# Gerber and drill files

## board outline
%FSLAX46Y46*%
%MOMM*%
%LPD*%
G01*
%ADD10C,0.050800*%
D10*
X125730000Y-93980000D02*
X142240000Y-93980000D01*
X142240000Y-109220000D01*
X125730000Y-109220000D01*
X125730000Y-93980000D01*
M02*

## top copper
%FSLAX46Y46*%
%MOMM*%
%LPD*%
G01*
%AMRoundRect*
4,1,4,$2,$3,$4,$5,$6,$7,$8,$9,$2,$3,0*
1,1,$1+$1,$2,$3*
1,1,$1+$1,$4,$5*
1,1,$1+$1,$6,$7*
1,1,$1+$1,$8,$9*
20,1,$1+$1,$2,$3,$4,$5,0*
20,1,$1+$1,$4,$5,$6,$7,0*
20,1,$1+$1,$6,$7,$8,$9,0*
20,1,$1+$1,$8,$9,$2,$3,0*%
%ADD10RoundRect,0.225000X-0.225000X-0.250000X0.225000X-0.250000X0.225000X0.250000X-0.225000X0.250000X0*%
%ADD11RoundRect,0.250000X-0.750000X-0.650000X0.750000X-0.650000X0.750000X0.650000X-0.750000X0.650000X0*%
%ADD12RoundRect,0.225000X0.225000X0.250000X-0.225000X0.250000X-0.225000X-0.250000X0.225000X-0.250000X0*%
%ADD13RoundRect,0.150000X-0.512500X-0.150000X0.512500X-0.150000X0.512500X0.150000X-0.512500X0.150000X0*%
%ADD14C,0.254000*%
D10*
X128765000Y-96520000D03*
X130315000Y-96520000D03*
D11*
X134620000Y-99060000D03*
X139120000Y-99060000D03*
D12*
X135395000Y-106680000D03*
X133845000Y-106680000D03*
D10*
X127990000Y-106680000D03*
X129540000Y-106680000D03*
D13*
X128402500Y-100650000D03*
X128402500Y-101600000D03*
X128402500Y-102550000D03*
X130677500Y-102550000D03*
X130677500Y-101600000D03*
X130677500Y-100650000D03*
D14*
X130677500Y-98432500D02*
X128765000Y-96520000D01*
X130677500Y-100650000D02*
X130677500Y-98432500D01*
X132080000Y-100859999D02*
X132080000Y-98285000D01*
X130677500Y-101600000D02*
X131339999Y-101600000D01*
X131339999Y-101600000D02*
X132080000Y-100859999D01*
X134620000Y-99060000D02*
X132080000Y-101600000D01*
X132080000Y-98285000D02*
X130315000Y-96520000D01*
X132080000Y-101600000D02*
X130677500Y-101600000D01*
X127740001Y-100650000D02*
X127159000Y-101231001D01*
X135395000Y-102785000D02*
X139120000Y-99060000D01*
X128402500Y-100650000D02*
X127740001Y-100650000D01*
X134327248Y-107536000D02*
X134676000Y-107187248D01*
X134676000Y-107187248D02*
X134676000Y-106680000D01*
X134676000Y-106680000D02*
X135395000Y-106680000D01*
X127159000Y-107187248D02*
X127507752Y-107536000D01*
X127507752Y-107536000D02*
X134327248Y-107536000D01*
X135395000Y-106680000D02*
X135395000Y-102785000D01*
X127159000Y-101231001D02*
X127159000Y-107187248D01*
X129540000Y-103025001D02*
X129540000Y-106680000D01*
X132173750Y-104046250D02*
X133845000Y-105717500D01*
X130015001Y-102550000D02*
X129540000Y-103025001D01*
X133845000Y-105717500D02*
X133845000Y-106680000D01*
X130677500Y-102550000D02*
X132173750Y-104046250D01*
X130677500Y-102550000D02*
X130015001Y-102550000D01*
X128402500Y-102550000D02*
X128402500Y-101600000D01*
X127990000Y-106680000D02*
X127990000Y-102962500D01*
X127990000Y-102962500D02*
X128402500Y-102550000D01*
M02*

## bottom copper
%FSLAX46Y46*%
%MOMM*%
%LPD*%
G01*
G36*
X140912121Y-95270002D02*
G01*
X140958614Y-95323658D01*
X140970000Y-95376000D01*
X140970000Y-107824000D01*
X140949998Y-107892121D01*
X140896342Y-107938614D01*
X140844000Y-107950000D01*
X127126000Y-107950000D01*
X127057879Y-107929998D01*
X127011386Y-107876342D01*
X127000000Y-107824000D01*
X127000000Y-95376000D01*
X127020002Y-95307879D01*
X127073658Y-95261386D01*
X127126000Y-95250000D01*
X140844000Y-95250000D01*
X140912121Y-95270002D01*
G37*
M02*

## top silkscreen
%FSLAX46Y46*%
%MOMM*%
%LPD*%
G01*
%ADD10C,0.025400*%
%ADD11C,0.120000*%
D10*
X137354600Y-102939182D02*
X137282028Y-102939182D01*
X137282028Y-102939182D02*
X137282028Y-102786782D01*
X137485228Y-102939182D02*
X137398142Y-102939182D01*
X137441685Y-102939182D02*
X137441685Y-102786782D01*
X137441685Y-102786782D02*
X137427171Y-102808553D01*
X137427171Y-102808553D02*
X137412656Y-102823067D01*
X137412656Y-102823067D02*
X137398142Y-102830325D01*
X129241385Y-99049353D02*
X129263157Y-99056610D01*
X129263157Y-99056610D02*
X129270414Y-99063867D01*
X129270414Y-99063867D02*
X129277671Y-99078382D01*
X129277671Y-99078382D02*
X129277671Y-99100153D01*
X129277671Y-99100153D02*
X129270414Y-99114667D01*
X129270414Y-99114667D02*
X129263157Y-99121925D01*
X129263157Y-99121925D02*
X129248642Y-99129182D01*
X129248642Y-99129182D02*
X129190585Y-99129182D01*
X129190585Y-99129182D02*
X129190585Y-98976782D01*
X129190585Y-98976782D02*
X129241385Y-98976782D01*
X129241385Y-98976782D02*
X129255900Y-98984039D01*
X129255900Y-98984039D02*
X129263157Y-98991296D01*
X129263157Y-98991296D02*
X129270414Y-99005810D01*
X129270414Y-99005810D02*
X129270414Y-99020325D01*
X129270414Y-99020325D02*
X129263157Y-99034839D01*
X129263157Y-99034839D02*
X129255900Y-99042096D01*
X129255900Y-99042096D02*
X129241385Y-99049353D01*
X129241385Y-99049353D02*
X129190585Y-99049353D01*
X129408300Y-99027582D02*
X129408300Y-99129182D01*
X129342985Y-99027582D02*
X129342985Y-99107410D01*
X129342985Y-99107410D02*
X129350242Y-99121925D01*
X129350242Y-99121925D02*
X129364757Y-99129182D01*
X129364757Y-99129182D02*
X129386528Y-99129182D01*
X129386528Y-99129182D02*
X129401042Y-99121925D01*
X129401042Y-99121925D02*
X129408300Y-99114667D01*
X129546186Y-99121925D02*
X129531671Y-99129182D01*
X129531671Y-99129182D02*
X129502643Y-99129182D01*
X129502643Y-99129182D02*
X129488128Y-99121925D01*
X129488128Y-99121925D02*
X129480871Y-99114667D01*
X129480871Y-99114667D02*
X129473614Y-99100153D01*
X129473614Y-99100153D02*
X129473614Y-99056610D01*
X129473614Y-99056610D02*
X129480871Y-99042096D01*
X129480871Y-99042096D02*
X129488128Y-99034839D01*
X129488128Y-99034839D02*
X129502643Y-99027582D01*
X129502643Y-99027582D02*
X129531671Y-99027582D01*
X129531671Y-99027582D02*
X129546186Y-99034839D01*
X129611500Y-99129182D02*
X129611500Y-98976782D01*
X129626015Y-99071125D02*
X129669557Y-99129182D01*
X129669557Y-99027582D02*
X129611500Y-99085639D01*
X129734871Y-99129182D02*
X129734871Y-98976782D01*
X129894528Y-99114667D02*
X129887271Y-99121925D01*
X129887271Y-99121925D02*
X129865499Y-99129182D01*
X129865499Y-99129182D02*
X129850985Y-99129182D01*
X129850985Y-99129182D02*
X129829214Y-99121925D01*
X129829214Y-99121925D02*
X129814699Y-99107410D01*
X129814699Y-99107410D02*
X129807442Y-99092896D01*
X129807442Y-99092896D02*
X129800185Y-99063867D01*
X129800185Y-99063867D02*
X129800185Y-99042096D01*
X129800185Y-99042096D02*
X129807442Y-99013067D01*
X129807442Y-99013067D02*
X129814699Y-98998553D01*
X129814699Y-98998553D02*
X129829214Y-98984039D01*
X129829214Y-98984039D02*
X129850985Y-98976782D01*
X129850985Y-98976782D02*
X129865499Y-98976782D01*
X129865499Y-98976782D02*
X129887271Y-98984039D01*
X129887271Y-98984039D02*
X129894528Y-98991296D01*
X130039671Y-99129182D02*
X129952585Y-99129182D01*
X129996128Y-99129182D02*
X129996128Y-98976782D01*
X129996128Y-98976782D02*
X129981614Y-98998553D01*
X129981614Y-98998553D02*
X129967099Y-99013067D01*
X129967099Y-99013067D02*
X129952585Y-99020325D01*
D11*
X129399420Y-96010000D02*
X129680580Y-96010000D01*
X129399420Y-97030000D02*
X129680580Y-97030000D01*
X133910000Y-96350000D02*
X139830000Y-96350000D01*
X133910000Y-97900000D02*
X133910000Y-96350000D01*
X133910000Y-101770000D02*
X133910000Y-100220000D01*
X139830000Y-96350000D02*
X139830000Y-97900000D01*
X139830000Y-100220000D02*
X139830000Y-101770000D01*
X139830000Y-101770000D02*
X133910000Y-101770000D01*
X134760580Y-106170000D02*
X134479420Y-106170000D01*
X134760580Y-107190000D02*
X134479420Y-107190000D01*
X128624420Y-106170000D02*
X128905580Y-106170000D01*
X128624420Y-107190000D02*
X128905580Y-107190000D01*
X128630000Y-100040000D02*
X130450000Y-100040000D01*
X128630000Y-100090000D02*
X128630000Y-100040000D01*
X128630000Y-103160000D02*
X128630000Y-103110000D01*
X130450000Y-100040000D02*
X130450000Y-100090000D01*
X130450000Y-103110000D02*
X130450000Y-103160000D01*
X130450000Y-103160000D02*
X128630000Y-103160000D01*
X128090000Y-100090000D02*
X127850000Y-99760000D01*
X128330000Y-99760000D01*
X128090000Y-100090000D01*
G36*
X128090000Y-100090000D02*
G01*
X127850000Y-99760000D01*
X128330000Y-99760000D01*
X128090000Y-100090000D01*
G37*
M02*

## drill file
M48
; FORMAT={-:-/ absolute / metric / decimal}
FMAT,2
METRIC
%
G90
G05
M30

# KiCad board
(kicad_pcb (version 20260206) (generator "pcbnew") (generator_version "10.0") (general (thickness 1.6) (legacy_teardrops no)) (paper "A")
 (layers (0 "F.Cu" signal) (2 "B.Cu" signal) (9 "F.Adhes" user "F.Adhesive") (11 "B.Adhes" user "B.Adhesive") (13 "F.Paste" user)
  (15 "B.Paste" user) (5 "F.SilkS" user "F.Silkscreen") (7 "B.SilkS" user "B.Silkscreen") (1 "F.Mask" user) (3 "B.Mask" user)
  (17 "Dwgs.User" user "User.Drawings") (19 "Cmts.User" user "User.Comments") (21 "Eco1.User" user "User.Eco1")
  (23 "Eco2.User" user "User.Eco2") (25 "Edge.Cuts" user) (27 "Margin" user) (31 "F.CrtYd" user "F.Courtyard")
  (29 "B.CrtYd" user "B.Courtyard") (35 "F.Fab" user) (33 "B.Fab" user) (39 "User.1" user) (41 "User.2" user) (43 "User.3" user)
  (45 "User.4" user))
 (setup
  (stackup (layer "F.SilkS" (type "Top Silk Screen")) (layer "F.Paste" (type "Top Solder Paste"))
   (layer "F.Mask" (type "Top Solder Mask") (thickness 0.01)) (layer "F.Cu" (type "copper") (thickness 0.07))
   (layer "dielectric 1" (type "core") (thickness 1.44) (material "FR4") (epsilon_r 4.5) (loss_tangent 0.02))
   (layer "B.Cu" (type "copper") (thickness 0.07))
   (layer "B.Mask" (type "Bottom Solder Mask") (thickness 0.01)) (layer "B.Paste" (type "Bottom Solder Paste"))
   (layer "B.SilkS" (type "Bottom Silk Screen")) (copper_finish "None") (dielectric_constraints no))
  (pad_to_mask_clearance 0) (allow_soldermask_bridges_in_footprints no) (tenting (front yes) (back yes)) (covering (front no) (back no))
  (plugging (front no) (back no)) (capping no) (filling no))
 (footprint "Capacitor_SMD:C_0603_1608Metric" (layer "F.Cu") (at 129.54 96.52)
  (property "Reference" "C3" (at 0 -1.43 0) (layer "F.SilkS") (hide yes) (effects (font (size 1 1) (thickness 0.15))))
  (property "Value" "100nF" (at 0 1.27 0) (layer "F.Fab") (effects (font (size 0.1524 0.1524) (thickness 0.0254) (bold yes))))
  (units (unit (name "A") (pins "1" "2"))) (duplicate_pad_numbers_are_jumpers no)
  (fp_line (start -0.14058 -0.51) (end 0.14058 -0.51) (stroke (width 0.12) (type solid)) (layer "F.SilkS"))
  (fp_line (start -0.14058 0.51) (end 0.14058 0.51) (stroke (width 0.12) (type solid)) (layer "F.SilkS"))
  (pad "1" smd roundrect (at -0.775 0) (size 0.9 0.95) (layers "F.Cu" "F.Mask" "F.Paste") (roundrect_rratio 0.25) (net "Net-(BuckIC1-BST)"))
  (pad "2" smd roundrect (at 0.775 0) (size 0.9 0.95) (layers "F.Cu" "F.Mask" "F.Paste") (roundrect_rratio 0.25) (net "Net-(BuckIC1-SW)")))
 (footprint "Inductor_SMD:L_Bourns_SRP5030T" (layer "F.Cu") (at 136.87 99.06)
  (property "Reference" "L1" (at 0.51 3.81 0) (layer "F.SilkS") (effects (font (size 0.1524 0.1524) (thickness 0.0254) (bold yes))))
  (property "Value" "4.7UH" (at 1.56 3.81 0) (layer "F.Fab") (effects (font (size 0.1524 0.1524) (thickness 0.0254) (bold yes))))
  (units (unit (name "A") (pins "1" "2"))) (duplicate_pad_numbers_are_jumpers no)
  (fp_line (start -2.96 -2.71) (end 2.96 -2.71) (stroke (width 0.12) (type solid)) (layer "F.SilkS"))
  (fp_line (start -2.96 -1.16) (end -2.96 -2.71) (stroke (width 0.12) (type solid)) (layer "F.SilkS"))
  (fp_line (start -2.96 2.71) (end -2.96 1.16) (stroke (width 0.12) (type solid)) (layer "F.SilkS"))
  (fp_line (start 2.96 -2.71) (end 2.96 -1.16) (stroke (width 0.12) (type solid)) (layer "F.SilkS"))
  (fp_line (start 2.96 1.16) (end 2.96 2.71) (stroke (width 0.12) (type solid)) (layer "F.SilkS"))
  (fp_line (start 2.96 2.71) (end -2.96 2.71) (stroke (width 0.12) (type solid)) (layer "F.SilkS"))
  (pad "1" smd roundrect (at -2.25 0) (size 2 1.8) (layers "F.Cu" "F.Mask" "F.Paste") (roundrect_rratio 0.138889) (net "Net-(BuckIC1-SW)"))
  (pad "2" smd roundrect (at 2.25 0) (size 2 1.8) (layers "F.Cu" "F.Mask" "F.Paste") (roundrect_rratio 0.138889) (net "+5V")))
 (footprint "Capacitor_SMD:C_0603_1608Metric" (layer "F.Cu") (at 134.62 106.68 180)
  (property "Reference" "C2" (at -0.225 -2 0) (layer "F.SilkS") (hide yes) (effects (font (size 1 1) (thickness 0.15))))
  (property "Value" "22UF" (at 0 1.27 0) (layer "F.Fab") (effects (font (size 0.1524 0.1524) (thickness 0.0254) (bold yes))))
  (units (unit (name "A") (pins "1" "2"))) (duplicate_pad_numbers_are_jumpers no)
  (fp_line (start -0.14058 0.51) (end 0.14058 0.51) (stroke (width 0.12) (type solid)) (layer "F.SilkS"))
  (fp_line (start -0.14058 -0.51) (end 0.14058 -0.51) (stroke (width 0.12) (type solid)) (layer "F.SilkS"))
  (pad "1" smd roundrect (at -0.775 0 180) (size 0.9 0.95) (layers "F.Cu" "F.Mask" "F.Paste") (roundrect_rratio 0.25) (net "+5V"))
  (pad "2" smd roundrect (at 0.775 0 180) (size 0.9 0.95) (layers "F.Cu" "F.Mask" "F.Paste") (roundrect_rratio 0.25) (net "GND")))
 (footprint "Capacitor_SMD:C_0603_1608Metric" (layer "F.Cu") (at 128.765 106.68)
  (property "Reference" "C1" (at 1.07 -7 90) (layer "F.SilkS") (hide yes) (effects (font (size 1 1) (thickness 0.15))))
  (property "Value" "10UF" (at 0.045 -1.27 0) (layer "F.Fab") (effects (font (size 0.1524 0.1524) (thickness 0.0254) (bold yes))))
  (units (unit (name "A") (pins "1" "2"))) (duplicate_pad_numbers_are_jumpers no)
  (fp_line (start -0.14058 -0.51) (end 0.14058 -0.51) (stroke (width 0.12) (type solid)) (layer "F.SilkS"))
  (fp_line (start -0.14058 0.51) (end 0.14058 0.51) (stroke (width 0.12) (type solid)) (layer "F.SilkS"))
  (pad "1" smd roundrect (at -0.775 0) (size 0.9 0.95) (layers "F.Cu" "F.Mask" "F.Paste") (roundrect_rratio 0.25) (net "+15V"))
  (pad "2" smd roundrect (at 0.775 0) (size 0.9 0.95) (layers "F.Cu" "F.Mask" "F.Paste") (roundrect_rratio 0.25) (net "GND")))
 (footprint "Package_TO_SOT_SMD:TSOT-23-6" (layer "F.Cu") (at 129.54 101.6)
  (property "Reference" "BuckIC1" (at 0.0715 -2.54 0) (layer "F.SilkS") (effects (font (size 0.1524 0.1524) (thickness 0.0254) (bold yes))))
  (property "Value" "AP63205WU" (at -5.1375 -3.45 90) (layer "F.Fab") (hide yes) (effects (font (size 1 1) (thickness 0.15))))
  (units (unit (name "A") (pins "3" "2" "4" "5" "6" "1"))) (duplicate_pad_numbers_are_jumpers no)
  (fp_line (start -0.91 -1.56) (end 0.91 -1.56) (stroke (width 0.12) (type solid)) (layer "F.SilkS"))
  (fp_line (start -0.91 -1.51) (end -0.91 -1.56) (stroke (width 0.12) (type solid)) (layer "F.SilkS"))
  (fp_line (start -0.91 1.56) (end -0.91 1.51) (stroke (width 0.12) (type solid)) (layer "F.SilkS"))
  (fp_line (start 0.91 -1.56) (end 0.91 -1.51) (stroke (width 0.12) (type solid)) (layer "F.SilkS"))
  (fp_line (start 0.91 1.51) (end 0.91 1.56) (stroke (width 0.12) (type solid)) (layer "F.SilkS"))
  (fp_line (start 0.91 1.56) (end -0.91 1.56) (stroke (width 0.12) (type solid)) (layer "F.SilkS"))
  (fp_poly (pts (xy -1.45 -1.51) (xy -1.69 -1.84) (xy -1.21 -1.84)) (stroke (width 0.12) (type solid)) (fill yes) (layer "F.SilkS"))
  (pad "1" smd roundrect (at -1.1375 -0.95) (size 1.325 0.6) (layers "F.Cu" "F.Mask" "F.Paste") (roundrect_rratio 0.25) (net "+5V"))
  (pad "2" smd roundrect (at -1.1375 0) (size 1.325 0.6) (layers "F.Cu" "F.Mask" "F.Paste") (roundrect_rratio 0.25) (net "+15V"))
  (pad "3" smd roundrect (at -1.1375 0.95) (size 1.325 0.6) (layers "F.Cu" "F.Mask" "F.Paste") (roundrect_rratio 0.25) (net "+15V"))
  (pad "4" smd roundrect (at 1.1375 0.95) (size 1.325 0.6) (layers "F.Cu" "F.Mask" "F.Paste") (roundrect_rratio 0.25) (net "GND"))
  (pad "5" smd roundrect (at 1.1375 0) (size 1.325 0.6) (layers "F.Cu" "F.Mask" "F.Paste") (roundrect_rratio 0.25) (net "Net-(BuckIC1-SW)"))
  (pad "6" smd roundrect (at 1.1375 -0.95) (size 1.325 0.6) (layers "F.Cu" "F.Mask" "F.Paste") (roundrect_rratio 0.25)
   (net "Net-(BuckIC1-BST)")))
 (gr_rect (start 125.73 93.98) (end 142.24 109.22) (stroke (width 0.0508) (type default)) (fill no) (layer "Edge.Cuts"))
 (segment (start 130.6775 98.4325) (end 128.765 96.52) (width 0.254) (layer "F.Cu") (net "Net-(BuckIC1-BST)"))
 (segment (start 130.6775 100.65) (end 130.6775 98.4325) (width 0.254) (layer "F.Cu") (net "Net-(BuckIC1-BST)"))
 (segment (start 132.08 100.859999) (end 132.08 98.285) (width 0.254) (layer "F.Cu") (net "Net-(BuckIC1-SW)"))
 (segment (start 130.6775 101.6) (end 131.339999 101.6) (width 0.254) (layer "F.Cu") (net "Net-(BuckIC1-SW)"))
 (segment (start 131.339999 101.6) (end 132.08 100.859999) (width 0.254) (layer "F.Cu") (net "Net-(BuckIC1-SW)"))
 (segment (start 134.62 99.06) (end 132.08 101.6) (width 0.254) (layer "F.Cu") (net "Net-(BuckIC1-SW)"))
 (segment (start 132.08 98.285) (end 130.315 96.52) (width 0.254) (layer "F.Cu") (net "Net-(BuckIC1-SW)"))
 (segment (start 132.08 101.6) (end 130.6775 101.6) (width 0.254) (layer "F.Cu") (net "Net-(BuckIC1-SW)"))
 (segment (start 127.740001 100.65) (end 127.159 101.231001) (width 0.254) (layer "F.Cu") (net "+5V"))
 (segment (start 135.395 102.785) (end 139.12 99.06) (width 0.254) (layer "F.Cu") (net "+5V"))
 (segment (start 128.4025 100.65) (end 127.740001 100.65) (width 0.254) (layer "F.Cu") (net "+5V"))
 (segment (start 134.327248 107.536) (end 134.676 107.187248) (width 0.254) (layer "F.Cu") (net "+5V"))
 (segment (start 134.676 107.187248) (end 134.676 106.68) (width 0.254) (layer "F.Cu") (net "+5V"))
 (segment (start 134.676 106.68) (end 135.395 106.68) (width 0.254) (layer "F.Cu") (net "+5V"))
 (segment (start 127.159 107.187248) (end 127.507752 107.536) (width 0.254) (layer "F.Cu") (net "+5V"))
 (segment (start 127.507752 107.536) (end 134.327248 107.536) (width 0.254) (layer "F.Cu") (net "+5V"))
 (segment (start 135.395 106.68) (end 135.395 102.785) (width 0.254) (layer "F.Cu") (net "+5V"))
 (segment (start 127.159 101.231001) (end 127.159 107.187248) (width 0.254) (layer "F.Cu") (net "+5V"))
 (segment (start 129.54 103.025001) (end 129.54 106.68) (width 0.254) (layer "F.Cu") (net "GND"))
 (segment (start 132.17375 104.04625) (end 133.845 105.7175) (width 0.254) (layer "F.Cu") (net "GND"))
 (segment (start 130.015001 102.55) (end 129.54 103.025001) (width 0.254) (layer "F.Cu") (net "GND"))
 (segment (start 133.845 105.7175) (end 133.845 106.68) (width 0.254) (layer "F.Cu") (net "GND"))
 (segment (start 130.6775 102.55) (end 132.17375 104.04625) (width 0.254) (layer "F.Cu") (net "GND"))
 (segment (start 130.6775 102.55) (end 130.015001 102.55) (width 0.254) (layer "F.Cu") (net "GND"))
 (segment (start 128.4025 102.55) (end 128.4025 101.6) (width 0.254) (layer "F.Cu") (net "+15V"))
 (segment (start 127.99 106.68) (end 127.99 102.9625) (width 0.254) (layer "F.Cu") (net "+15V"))
 (segment (start 127.99 102.9625) (end 128.4025 102.55) (width 0.254) (layer "F.Cu") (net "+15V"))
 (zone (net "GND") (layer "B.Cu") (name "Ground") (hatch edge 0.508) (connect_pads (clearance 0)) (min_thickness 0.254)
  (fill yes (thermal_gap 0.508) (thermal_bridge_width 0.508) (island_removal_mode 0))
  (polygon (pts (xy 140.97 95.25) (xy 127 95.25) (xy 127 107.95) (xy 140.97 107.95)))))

